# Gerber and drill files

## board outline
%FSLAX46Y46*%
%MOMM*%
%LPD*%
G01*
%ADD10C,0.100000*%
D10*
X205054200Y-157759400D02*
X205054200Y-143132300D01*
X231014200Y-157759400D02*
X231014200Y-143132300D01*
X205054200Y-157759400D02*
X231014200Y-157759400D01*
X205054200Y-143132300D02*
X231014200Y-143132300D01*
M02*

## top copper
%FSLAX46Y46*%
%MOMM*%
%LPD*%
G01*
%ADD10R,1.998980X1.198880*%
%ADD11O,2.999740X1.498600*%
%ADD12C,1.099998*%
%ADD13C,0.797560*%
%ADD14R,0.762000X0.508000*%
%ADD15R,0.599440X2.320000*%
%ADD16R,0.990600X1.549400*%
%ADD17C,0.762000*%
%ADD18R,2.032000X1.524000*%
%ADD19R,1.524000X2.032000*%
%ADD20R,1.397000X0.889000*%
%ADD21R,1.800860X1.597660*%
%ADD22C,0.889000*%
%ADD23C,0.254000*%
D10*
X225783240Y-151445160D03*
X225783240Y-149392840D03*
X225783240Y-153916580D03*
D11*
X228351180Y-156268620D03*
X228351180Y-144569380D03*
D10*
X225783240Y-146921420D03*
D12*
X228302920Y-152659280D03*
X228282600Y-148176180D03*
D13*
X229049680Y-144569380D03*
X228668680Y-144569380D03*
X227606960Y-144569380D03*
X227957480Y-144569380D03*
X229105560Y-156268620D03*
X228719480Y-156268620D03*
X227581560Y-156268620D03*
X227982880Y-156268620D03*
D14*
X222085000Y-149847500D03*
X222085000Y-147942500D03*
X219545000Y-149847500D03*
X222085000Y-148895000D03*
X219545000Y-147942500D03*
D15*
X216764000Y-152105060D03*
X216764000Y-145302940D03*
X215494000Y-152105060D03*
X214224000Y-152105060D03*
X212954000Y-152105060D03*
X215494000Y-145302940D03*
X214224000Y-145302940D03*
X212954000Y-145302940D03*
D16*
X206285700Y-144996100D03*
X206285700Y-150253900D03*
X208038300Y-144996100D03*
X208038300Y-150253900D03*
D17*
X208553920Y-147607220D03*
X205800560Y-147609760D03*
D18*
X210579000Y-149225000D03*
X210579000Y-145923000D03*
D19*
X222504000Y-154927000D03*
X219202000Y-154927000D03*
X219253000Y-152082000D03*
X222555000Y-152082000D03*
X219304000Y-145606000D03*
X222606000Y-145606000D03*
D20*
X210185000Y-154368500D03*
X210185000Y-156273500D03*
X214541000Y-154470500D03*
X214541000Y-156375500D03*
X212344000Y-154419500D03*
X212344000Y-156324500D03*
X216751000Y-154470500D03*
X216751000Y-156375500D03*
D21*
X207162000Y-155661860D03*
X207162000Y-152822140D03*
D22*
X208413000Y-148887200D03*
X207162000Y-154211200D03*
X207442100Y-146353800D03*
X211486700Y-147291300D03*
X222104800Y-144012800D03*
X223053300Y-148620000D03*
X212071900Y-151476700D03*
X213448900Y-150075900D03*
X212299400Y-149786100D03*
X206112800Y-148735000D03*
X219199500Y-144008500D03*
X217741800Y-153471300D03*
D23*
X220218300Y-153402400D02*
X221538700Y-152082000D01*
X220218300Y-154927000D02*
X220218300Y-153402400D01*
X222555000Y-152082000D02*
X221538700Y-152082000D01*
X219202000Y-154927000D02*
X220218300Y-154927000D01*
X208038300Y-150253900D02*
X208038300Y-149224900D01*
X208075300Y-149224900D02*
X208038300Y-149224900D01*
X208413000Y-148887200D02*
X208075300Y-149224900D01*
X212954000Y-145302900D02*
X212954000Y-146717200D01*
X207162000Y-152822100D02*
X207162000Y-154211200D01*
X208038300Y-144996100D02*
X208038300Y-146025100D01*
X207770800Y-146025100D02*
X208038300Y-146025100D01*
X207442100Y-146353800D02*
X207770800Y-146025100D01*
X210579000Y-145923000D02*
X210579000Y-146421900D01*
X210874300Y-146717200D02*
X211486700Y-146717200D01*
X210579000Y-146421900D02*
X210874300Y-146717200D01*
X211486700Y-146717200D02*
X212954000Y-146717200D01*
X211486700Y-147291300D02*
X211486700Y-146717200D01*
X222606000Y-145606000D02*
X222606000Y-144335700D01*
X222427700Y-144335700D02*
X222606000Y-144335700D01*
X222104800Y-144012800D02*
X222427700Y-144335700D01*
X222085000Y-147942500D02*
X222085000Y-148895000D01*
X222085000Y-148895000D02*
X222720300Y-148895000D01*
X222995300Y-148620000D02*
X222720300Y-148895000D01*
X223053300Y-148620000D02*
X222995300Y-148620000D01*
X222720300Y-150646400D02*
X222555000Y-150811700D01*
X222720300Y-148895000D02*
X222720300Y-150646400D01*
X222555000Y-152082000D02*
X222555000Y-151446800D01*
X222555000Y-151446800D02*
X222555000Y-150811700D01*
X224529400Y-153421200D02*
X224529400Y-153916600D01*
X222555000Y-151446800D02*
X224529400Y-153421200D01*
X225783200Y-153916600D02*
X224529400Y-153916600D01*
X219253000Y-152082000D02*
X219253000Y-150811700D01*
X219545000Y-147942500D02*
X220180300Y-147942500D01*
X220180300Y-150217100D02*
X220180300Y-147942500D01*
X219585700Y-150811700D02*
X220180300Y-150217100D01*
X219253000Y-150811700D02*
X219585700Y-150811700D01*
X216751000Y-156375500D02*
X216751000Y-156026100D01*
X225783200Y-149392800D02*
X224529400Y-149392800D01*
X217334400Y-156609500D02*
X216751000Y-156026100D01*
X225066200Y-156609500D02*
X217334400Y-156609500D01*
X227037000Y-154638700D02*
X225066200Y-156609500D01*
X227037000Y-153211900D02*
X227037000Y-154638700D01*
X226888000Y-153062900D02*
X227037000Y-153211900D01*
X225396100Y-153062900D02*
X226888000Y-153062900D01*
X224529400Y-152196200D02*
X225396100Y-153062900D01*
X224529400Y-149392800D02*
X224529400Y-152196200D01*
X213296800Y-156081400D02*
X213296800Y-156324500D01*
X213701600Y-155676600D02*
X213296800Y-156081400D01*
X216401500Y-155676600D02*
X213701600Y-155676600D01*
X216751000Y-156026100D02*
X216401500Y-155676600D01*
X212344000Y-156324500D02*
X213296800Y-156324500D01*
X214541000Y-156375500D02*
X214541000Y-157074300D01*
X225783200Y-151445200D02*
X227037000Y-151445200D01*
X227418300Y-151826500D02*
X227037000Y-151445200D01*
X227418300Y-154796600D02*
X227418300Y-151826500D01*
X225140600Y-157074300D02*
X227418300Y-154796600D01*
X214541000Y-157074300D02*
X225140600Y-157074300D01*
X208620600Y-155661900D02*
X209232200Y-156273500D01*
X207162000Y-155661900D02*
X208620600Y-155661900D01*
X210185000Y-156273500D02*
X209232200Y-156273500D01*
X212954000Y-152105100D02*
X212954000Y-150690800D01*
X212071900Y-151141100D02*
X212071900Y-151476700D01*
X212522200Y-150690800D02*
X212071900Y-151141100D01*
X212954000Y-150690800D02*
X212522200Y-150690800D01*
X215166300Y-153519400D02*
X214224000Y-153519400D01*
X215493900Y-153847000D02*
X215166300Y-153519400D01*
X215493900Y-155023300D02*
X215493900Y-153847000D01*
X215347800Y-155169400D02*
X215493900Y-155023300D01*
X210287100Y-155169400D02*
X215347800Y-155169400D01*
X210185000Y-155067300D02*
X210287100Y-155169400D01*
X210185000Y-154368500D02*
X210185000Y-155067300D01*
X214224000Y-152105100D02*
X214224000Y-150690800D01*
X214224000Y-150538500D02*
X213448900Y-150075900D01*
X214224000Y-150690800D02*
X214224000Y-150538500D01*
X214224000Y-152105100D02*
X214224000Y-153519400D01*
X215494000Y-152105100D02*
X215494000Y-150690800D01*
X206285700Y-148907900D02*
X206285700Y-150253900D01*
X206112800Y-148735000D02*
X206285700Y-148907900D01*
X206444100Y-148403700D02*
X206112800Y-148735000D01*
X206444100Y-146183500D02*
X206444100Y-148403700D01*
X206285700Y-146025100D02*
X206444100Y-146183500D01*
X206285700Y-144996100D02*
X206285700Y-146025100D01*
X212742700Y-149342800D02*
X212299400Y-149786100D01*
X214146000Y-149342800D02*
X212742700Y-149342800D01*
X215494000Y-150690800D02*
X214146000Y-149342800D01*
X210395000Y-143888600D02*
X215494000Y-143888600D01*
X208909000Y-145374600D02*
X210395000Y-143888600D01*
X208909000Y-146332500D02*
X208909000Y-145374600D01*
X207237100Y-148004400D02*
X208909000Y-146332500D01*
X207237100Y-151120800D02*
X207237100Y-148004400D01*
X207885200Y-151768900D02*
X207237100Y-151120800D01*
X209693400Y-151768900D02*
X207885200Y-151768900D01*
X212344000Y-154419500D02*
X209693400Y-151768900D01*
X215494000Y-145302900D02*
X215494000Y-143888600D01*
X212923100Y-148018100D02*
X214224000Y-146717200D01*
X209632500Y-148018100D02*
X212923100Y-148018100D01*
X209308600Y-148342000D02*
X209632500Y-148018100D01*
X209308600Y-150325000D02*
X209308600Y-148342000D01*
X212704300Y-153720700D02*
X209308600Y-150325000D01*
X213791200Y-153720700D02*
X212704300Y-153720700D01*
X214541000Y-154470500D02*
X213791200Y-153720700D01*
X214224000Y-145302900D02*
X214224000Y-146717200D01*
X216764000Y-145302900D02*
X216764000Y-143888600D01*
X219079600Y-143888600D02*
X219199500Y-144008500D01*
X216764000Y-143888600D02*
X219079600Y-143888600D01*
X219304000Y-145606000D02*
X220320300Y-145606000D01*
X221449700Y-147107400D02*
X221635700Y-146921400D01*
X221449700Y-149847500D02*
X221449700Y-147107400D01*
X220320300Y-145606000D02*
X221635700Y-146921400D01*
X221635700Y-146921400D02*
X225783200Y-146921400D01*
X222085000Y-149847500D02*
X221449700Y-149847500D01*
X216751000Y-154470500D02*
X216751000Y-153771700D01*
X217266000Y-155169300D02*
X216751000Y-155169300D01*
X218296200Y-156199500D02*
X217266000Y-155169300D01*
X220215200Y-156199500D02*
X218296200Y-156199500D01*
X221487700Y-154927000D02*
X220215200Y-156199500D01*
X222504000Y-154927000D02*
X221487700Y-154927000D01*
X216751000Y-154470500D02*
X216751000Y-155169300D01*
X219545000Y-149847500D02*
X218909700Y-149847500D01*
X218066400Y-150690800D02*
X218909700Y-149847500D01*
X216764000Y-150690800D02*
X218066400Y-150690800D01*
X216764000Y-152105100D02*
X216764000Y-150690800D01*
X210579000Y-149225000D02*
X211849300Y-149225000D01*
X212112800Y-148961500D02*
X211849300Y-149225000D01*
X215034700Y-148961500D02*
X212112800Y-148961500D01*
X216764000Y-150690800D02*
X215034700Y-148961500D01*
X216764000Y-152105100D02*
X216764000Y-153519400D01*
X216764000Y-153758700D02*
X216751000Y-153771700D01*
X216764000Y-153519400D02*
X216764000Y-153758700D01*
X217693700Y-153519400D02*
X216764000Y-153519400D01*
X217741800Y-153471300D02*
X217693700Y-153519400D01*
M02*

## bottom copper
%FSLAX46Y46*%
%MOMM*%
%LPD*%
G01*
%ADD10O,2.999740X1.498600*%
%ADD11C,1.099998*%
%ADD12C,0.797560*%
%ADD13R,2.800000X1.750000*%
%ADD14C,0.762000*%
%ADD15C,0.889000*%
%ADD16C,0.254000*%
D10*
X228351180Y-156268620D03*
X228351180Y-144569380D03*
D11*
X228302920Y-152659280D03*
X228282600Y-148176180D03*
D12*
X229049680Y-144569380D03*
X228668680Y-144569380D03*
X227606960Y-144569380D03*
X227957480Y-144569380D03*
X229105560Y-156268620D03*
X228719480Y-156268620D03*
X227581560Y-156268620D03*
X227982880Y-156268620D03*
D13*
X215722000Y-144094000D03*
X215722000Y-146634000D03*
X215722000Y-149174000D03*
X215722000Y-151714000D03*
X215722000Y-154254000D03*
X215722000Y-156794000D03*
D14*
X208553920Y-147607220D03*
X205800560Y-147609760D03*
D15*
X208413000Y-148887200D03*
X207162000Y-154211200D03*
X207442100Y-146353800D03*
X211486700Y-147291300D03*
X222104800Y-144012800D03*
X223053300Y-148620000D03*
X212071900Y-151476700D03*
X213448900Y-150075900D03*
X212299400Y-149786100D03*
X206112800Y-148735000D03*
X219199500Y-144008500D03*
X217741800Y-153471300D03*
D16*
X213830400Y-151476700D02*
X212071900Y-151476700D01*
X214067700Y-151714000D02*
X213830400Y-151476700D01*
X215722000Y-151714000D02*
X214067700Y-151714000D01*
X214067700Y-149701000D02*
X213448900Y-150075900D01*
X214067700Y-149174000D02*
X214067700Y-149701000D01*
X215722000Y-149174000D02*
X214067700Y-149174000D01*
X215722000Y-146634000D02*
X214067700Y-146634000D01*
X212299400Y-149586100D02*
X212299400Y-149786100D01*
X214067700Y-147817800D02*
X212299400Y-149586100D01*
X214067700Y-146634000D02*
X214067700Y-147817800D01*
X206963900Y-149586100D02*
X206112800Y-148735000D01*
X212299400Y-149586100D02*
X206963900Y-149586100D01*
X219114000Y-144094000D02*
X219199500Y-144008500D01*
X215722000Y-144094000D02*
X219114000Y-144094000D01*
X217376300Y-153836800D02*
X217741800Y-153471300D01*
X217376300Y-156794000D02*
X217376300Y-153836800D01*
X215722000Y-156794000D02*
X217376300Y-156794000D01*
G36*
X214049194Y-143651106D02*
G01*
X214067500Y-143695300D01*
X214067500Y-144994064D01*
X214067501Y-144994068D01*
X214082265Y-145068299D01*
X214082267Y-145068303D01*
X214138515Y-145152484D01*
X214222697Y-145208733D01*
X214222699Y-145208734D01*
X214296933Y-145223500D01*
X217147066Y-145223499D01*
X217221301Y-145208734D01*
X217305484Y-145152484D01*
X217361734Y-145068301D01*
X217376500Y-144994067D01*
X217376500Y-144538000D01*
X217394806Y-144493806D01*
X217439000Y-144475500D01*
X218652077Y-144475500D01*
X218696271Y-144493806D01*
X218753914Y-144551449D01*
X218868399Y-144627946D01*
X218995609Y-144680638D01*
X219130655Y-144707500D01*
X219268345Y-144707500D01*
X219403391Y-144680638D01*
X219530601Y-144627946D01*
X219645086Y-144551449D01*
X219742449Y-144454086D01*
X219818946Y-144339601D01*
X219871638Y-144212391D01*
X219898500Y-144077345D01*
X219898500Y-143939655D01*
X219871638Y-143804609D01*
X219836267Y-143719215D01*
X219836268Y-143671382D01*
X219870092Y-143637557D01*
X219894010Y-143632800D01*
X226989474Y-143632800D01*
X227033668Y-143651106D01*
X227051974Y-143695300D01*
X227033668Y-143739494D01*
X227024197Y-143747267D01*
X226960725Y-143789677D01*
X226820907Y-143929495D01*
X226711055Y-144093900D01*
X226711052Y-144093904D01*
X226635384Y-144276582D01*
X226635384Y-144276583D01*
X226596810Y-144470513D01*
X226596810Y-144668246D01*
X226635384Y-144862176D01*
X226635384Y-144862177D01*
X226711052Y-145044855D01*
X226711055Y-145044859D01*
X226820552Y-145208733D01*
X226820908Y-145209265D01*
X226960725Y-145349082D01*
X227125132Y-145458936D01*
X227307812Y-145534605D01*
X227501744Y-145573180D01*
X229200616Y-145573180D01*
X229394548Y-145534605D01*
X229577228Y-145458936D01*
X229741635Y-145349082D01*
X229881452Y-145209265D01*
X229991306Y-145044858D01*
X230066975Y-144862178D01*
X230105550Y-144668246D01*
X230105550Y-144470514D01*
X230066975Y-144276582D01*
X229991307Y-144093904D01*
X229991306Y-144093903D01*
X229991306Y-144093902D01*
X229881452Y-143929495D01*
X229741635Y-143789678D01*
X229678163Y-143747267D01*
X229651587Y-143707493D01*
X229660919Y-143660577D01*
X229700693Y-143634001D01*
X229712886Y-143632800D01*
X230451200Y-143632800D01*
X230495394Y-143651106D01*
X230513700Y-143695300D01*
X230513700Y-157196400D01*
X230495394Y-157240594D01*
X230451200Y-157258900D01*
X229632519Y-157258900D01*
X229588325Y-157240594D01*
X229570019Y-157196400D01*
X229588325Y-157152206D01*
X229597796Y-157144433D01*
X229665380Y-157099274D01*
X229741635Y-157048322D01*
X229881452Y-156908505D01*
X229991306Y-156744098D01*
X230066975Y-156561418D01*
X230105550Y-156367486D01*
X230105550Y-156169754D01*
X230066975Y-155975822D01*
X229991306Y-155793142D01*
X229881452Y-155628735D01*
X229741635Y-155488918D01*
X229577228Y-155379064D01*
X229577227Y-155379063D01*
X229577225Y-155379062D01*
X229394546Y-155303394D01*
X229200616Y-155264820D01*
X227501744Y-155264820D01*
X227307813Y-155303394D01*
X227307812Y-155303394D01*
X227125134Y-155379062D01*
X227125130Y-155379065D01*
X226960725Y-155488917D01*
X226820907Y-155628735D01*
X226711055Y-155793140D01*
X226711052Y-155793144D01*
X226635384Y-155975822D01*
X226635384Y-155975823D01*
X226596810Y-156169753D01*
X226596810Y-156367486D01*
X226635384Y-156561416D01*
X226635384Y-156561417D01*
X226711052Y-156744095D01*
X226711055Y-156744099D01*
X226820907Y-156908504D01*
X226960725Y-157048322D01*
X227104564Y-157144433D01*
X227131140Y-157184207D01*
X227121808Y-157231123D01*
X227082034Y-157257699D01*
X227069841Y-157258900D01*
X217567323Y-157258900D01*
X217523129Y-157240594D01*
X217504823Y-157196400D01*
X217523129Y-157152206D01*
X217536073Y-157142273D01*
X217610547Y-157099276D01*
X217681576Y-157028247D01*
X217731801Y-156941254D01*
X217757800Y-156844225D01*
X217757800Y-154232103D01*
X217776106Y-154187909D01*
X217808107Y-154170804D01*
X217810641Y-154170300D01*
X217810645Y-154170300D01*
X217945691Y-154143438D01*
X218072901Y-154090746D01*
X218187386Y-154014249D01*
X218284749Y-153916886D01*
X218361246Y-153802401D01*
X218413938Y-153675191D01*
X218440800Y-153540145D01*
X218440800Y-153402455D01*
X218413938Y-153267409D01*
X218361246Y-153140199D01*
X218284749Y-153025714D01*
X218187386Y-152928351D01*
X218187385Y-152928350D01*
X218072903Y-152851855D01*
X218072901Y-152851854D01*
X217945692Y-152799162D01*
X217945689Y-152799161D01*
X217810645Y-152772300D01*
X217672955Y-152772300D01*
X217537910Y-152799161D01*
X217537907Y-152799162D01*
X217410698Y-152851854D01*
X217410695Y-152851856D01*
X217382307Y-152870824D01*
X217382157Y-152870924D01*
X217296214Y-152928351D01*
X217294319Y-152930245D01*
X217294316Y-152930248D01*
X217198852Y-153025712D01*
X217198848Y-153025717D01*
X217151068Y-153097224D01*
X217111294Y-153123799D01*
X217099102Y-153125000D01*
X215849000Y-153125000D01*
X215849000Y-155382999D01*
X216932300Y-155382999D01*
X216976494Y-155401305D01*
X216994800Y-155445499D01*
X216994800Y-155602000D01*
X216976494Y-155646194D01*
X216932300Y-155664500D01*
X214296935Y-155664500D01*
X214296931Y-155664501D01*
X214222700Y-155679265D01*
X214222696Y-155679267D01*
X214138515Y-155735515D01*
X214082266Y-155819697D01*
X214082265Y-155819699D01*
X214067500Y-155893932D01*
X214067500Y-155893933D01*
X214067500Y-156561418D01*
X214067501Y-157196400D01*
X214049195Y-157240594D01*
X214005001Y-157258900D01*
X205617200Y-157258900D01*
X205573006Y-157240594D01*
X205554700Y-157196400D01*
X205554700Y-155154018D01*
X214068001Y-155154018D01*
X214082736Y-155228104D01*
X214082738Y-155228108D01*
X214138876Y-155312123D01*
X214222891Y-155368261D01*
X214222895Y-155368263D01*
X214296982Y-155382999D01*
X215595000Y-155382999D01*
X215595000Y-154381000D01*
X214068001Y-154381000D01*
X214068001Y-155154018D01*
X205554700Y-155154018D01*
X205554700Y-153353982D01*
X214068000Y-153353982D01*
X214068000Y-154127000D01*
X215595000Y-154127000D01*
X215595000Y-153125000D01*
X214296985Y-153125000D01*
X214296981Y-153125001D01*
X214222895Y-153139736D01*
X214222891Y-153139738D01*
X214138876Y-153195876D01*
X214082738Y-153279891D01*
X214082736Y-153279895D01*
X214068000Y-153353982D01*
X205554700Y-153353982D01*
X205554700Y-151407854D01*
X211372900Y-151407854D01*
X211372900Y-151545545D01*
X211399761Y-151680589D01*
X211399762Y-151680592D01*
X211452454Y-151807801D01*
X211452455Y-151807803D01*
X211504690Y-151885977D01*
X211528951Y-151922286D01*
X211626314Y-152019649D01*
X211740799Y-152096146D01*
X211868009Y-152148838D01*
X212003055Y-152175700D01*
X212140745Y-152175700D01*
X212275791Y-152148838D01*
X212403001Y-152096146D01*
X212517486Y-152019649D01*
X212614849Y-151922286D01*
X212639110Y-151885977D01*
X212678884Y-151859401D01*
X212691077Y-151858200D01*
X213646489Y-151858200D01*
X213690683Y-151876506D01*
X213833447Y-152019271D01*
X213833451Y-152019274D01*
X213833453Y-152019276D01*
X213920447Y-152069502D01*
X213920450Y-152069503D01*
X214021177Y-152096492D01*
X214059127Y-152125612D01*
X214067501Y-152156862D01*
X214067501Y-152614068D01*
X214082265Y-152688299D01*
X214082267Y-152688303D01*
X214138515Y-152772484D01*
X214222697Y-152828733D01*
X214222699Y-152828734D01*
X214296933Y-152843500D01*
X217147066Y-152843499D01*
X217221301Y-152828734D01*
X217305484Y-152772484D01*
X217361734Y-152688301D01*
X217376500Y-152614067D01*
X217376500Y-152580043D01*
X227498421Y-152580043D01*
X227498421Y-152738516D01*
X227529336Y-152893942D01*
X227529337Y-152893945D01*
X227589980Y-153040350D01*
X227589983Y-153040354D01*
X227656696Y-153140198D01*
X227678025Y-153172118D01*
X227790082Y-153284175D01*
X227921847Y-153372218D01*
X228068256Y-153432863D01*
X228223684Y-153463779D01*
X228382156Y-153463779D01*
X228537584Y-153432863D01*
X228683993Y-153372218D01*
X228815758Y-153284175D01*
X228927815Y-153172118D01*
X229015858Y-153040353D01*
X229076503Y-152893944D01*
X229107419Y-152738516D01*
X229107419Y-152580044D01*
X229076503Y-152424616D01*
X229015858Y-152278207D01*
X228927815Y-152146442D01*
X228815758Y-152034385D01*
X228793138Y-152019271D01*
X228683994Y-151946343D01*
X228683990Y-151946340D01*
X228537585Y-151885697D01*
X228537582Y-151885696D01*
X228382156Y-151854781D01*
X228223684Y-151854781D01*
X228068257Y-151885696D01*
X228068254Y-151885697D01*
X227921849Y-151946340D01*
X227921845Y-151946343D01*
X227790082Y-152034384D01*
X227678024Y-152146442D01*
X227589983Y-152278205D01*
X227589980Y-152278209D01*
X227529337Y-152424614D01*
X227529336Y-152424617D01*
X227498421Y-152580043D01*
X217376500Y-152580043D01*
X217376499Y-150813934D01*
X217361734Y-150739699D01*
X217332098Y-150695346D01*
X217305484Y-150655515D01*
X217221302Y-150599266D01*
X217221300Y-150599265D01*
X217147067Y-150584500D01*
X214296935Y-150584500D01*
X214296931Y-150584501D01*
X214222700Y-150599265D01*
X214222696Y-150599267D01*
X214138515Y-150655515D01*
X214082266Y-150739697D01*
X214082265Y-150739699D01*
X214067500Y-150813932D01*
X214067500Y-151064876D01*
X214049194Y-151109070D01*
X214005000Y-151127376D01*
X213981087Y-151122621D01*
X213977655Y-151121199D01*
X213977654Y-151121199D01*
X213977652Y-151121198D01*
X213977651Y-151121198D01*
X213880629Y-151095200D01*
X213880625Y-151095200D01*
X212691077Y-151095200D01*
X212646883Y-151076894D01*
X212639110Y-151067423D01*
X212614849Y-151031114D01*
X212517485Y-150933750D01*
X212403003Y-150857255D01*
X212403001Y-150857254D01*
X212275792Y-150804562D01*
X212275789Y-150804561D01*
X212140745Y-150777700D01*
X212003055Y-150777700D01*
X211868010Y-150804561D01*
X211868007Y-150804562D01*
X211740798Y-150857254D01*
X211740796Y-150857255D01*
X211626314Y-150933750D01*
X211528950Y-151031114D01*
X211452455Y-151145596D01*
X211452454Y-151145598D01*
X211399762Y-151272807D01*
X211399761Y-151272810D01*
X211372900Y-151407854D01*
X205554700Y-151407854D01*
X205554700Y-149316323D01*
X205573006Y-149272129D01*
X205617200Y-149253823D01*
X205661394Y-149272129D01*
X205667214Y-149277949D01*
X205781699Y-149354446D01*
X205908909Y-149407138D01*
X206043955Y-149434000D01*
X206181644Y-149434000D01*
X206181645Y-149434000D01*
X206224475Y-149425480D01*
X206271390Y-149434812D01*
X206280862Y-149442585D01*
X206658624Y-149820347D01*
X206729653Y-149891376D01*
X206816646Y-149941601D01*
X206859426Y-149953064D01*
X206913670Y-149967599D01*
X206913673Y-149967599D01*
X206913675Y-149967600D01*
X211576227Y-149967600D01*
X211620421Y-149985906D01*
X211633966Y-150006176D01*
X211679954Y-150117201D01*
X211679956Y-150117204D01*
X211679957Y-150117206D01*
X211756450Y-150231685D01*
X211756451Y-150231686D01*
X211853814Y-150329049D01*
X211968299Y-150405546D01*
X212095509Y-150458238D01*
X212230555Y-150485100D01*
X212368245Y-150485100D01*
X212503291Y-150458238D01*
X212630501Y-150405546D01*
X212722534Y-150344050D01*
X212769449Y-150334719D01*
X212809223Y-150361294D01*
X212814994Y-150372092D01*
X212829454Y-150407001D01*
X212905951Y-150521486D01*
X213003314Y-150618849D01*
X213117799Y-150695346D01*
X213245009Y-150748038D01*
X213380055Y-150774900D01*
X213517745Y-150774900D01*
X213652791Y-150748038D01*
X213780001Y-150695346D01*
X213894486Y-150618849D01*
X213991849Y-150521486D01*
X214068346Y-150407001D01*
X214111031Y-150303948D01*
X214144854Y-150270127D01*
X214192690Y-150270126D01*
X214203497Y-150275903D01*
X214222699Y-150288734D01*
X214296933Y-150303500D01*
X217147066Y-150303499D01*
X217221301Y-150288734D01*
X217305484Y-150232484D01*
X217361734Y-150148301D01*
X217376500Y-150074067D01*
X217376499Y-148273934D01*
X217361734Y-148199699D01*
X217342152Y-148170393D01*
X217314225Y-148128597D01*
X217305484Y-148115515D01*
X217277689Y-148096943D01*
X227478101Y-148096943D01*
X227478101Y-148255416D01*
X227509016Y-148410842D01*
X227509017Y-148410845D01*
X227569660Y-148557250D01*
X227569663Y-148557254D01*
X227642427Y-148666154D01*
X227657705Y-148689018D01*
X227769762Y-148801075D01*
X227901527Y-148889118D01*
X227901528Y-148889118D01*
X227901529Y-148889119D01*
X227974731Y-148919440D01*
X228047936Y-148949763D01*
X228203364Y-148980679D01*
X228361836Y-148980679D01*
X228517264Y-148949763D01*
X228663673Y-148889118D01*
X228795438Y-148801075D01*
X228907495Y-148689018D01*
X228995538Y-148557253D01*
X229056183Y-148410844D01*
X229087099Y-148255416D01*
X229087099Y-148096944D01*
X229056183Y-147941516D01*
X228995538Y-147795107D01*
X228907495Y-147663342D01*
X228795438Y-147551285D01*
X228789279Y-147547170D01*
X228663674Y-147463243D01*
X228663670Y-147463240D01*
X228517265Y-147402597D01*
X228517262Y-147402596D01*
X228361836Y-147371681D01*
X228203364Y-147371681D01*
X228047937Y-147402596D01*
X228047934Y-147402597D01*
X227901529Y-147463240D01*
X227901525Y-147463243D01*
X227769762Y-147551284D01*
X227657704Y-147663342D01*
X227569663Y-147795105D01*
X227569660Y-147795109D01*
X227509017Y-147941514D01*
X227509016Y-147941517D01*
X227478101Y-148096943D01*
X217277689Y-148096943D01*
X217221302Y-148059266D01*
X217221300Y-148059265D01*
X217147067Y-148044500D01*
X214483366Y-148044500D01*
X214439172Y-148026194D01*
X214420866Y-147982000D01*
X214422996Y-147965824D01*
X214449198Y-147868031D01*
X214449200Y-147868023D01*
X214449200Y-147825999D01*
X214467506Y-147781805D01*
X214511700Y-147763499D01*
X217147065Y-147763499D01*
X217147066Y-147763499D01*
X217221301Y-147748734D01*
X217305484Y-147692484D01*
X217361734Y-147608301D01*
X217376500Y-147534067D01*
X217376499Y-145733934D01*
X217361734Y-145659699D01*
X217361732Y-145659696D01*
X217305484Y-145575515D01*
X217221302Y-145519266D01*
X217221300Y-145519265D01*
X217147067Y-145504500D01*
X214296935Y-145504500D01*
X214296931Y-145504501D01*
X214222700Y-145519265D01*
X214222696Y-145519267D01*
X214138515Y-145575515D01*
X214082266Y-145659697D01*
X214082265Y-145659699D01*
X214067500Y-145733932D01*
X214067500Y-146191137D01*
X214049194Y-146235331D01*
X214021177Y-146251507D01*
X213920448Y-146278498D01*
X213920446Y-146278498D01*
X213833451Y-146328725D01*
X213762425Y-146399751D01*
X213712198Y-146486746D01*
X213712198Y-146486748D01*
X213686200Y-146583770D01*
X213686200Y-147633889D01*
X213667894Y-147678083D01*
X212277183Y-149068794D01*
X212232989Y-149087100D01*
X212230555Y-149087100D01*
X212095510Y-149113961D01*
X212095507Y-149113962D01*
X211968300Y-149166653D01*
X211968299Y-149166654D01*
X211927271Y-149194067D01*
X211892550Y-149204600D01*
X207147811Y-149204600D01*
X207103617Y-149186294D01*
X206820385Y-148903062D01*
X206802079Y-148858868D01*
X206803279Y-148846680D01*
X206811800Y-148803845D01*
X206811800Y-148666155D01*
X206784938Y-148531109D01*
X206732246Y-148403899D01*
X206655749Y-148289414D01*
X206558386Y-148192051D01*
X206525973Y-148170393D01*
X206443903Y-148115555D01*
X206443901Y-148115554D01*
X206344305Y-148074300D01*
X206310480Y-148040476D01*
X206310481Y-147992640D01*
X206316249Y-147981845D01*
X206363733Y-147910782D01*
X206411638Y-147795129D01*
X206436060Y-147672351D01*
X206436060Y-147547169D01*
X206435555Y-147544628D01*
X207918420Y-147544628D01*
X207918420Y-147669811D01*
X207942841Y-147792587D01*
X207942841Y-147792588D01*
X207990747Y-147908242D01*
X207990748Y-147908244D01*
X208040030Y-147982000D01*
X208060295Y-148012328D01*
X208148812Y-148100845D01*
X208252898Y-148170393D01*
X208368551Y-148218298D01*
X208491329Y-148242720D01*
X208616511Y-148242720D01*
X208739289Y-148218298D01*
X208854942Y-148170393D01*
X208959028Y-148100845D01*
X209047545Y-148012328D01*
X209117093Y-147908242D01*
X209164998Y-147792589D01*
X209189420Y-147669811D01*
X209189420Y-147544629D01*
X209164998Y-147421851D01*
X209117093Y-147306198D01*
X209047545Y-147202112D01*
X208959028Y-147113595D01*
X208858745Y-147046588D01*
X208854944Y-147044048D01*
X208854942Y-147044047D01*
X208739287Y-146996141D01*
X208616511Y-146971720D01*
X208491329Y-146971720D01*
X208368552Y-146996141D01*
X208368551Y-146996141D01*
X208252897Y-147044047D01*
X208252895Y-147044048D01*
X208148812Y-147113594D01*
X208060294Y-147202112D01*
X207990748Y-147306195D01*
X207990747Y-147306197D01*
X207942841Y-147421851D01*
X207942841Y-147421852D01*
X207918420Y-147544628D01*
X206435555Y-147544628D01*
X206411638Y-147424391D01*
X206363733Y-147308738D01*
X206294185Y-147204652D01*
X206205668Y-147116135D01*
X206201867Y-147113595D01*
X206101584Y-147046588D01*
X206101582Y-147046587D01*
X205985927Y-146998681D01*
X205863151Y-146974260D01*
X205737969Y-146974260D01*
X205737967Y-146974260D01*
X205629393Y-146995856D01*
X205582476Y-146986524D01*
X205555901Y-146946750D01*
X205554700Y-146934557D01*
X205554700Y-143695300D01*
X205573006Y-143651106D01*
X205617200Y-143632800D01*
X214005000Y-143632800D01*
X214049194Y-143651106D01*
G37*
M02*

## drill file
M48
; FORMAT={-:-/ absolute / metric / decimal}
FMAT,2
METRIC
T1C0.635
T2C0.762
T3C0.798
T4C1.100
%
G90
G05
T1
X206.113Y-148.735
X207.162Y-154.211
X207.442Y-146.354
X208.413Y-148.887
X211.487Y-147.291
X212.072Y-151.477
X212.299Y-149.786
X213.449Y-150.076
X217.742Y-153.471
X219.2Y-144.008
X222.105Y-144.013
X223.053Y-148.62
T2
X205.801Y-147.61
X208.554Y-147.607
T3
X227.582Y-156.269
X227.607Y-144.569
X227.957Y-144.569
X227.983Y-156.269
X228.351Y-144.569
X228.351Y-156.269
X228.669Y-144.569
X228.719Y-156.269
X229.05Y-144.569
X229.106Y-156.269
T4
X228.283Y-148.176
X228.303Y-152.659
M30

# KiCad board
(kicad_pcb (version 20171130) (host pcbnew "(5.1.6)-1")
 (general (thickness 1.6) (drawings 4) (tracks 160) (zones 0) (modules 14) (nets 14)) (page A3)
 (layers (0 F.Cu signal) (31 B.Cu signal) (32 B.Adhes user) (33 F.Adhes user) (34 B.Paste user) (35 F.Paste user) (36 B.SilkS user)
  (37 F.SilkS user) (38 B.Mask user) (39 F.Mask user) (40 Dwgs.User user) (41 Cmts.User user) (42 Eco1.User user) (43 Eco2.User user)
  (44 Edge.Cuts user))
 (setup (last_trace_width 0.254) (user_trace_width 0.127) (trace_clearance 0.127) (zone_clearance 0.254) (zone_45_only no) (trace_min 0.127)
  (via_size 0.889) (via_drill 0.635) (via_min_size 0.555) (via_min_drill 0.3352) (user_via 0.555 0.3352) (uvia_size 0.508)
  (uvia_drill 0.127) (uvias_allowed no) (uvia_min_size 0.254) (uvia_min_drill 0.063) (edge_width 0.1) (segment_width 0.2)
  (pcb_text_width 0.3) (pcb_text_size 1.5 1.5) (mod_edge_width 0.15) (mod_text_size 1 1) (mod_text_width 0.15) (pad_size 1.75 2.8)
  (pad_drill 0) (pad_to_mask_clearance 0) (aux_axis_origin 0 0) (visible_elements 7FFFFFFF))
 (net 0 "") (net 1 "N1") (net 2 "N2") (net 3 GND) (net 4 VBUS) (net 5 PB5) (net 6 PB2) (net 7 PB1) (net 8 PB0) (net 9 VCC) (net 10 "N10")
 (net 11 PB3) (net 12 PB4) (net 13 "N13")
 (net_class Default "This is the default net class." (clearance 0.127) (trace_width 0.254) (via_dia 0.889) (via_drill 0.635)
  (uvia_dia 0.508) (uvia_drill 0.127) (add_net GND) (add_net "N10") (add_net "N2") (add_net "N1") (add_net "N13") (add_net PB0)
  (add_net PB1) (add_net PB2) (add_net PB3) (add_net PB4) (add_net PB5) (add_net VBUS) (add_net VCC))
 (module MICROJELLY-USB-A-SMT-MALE (layer F.Cu) (at 229.451 150.419 270)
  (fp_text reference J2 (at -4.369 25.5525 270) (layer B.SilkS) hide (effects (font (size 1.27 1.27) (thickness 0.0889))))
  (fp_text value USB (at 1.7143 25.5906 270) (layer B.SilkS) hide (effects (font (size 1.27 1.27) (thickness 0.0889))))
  (pad 2 smd rect (at 1.02616 3.66776 270) (size 1.19888 1.99898) (layers F.Cu F.Paste F.Mask) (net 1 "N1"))
  (pad 3 smd rect (at -1.02616 3.66776 270) (size 1.19888 1.99898) (layers F.Cu F.Paste F.Mask) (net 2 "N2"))
  (pad 1 smd rect (at 3.49758 3.66776 270) (size 1.19888 1.99898) (layers F.Cu F.Paste F.Mask) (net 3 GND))
  (pad P$1 thru_hole oval (at 5.84962 1.09982 270) (size 1.4986 2.99974) (drill 0.79756) (layers *.Cu *.Mask F.Paste F.SilkS))
  (pad P$3 thru_hole oval (at -5.84962 1.09982 270) (size 1.4986 2.99974) (drill 0.79756) (layers *.Cu *.Mask F.Paste F.SilkS))
  (pad 4 smd rect (at -3.49758 3.66776 270) (size 1.19888 1.99898) (layers F.Cu F.Paste F.Mask) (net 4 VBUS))
  (pad P$4 thru_hole circle (at 2.24028 1.14808 270) (size 1.099998 1.099998) (drill 1.099998) (layers *.Cu *.Mask F.SilkS))
  (pad P$5 thru_hole circle (at -2.24282 1.1684 270) (size 1.099998 1.099998) (drill 1.099998) (layers *.Cu *.Mask F.SilkS))
  (pad P$4 thru_hole circle (at -5.84962 0.40132 270) (size 0.79756 0.79756) (drill 0.79756) (layers *.Cu F.Paste F.SilkS F.Mask))
  (pad P$5 thru_hole circle (at -5.84962 0.78232 270) (size 0.79756 0.79756) (drill 0.79756) (layers *.Cu F.Paste F.SilkS F.Mask))
  (pad P$6 thru_hole circle (at -5.84962 1.84404 270) (size 0.79756 0.79756) (drill 0.79756) (layers *.Cu F.Paste F.SilkS F.Mask))
  (pad P$7 thru_hole circle (at -5.84962 1.49352 270) (size 0.79756 0.79756) (drill 0.79756) (layers *.Cu F.Paste F.SilkS F.Mask))
  (pad P$2 thru_hole circle (at 5.84962 0.34544 270) (size 0.79756 0.79756) (drill 0.79756) (layers *.Cu F.Paste F.SilkS F.Mask))
  (pad P$3 thru_hole circle (at 5.84962 0.73152 270) (size 0.79756 0.79756) (drill 0.79756) (layers *.Cu F.Paste F.SilkS F.Mask))
  (pad P$4 thru_hole circle (at 5.84962 1.86944 270) (size 0.79756 0.79756) (drill 0.79756) (layers *.Cu F.Paste F.SilkS F.Mask))
  (pad P$5 thru_hole circle (at 5.84962 1.46812 270) (size 0.79756 0.79756) (drill 0.79756) (layers *.Cu F.Paste F.SilkS F.Mask)))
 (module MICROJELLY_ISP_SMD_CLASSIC (layer B.Cu) (at 213.944 150.444 270)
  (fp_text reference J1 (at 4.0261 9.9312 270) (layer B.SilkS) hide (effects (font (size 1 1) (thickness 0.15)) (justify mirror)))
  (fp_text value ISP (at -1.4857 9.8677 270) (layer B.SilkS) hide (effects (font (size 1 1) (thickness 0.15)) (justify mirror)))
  (pad 5 smd rect (at -6.35 -1.778 270) (size 1.75 2.8) (layers B.Cu B.Paste B.Mask) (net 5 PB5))
  (pad 3 smd rect (at -3.81 -1.778 270) (size 1.75 2.8) (layers B.Cu B.Paste B.Mask) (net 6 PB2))
  (pad 1 smd rect (at -1.27 -1.778 270) (size 1.75 2.8) (layers B.Cu B.Paste B.Mask) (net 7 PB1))
  (pad 4 smd rect (at 1.27 -1.778 270) (size 1.75 2.8) (layers B.Cu B.Paste B.Mask) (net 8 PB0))
  (pad 6 smd rect (at 3.81 -1.778 270) (size 1.75 2.8) (layers B.Cu B.Paste B.Mask) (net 3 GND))
  (pad 2 smd rect (at 6.35 -1.778 270) (size 1.75 2.8) (layers B.Cu B.Paste B.Mask) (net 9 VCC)))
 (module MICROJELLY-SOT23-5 (layer F.Cu) (at 220.815 148.895 90)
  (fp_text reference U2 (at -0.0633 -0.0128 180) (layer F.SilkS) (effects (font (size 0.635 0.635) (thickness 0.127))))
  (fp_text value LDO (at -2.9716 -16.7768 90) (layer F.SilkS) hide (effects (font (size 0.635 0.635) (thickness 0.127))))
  (pad 1 smd rect (at -0.9525 1.27 90) (size 0.508 0.762) (layers F.Cu F.Paste F.Mask) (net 4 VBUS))
  (pad 3 smd rect (at 0.9525 1.27 90) (size 0.508 0.762) (layers F.Cu F.Paste F.Mask) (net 3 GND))
  (pad 5 smd rect (at -0.9525 -1.27 90) (size 0.508 0.762) (layers F.Cu F.Paste F.Mask) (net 9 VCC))
  (pad 2 smd rect (at 0 1.27 90) (size 0.508 0.762) (layers F.Cu F.Paste F.Mask) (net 3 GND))
  (pad 4 smd rect (at 0.9525 -1.27 90) (size 0.508 0.762) (layers F.Cu F.Paste F.Mask) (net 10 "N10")))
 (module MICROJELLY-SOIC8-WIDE (layer F.Cu) (at 214.859 148.704 180)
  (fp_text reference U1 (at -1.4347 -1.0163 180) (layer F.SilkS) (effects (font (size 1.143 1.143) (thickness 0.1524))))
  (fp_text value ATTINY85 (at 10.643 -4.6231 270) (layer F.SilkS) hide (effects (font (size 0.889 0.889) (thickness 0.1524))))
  (pad 8 smd rect (at -1.905 -3.40106 180) (size 0.59944 2.32) (layers F.Cu F.Paste F.Mask) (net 9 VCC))
  (pad 1 smd rect (at -1.905 3.40106 180) (size 0.59944 2.32) (layers F.Cu F.Paste F.Mask) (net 5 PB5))
  (pad 7 smd rect (at -0.635 -3.40106 180) (size 0.59944 2.32) (layers F.Cu F.Paste F.Mask) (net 6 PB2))
  (pad 6 smd rect (at 0.635 -3.40106 180) (size 0.59944 2.32) (layers F.Cu F.Paste F.Mask) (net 7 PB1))
  (pad 5 smd rect (at 1.905 -3.40106 180) (size 0.59944 2.32) (layers F.Cu F.Paste F.Mask) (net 8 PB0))
  (pad 2 smd rect (at -0.635 3.40106 180) (size 0.59944 2.32) (layers F.Cu F.Paste F.Mask) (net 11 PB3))
  (pad 3 smd rect (at 0.635 3.40106 180) (size 0.59944 2.32) (layers F.Cu F.Paste F.Mask) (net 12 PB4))
  (pad 4 smd rect (at 1.905 3.40106 180) (size 0.59944 2.32) (layers F.Cu F.Paste F.Mask) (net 3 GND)))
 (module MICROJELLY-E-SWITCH (layer F.Cu) (at 207.162 147.625 270)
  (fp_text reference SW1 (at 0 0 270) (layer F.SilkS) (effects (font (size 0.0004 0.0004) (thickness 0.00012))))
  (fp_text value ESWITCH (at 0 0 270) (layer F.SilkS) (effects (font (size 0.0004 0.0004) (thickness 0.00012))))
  (pad 1 smd rect (at -2.6289 0.8763 270) (size 1.5494 0.9906) (layers F.Cu F.Paste F.Mask) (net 6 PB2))
  (pad 1 smd rect (at 2.6289 0.8763 270) (size 1.5494 0.9906) (layers F.Cu F.Paste F.Mask) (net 6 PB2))
  (pad 2 smd rect (at -2.6289 -0.8763 270) (size 1.5494 0.9906) (layers F.Cu F.Paste F.Mask) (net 3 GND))
  (pad 2 smd rect (at 2.6289 -0.8763 270) (size 1.5494 0.9906) (layers F.Cu F.Paste F.Mask) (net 3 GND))
  (pad P$5 thru_hole circle (at -0.01778 -1.39192 270) (size 0.762 0.762) (drill 0.762) (layers *.Cu *.Mask F.SilkS))
  (pad P$6 thru_hole circle (at -0.01524 1.36144 270) (size 0.762 0.762) (drill 0.762) (layers *.Cu *.Mask F.SilkS)))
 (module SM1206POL (layer F.Cu) (at 210.579 147.574 90)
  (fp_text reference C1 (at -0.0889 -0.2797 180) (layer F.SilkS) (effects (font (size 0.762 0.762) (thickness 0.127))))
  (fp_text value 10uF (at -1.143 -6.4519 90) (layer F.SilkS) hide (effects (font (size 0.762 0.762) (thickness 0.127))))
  (pad 1 smd rect (at -1.651 0 90) (size 1.524 2.032) (layers F.Cu F.Paste F.Mask) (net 9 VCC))
  (pad 2 smd rect (at 1.651 0 90) (size 1.524 2.032) (layers F.Cu F.Paste F.Mask) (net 3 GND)))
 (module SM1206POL (layer F.Cu) (at 220.853 154.927 180)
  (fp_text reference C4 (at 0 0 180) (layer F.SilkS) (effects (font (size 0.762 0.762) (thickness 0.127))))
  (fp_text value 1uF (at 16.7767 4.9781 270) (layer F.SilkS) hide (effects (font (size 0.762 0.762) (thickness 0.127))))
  (pad 1 smd rect (at -1.651 0 180) (size 1.524 2.032) (layers F.Cu F.Paste F.Mask) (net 9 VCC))
  (pad 2 smd rect (at 1.651 0 180) (size 1.524 2.032) (layers F.Cu F.Paste F.Mask) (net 3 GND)))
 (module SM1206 (layer F.Cu) (at 220.904 152.082)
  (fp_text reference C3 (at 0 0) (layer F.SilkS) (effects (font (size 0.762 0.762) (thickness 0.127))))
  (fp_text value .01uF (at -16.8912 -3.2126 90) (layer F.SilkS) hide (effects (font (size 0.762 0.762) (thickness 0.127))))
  (pad 1 smd rect (at -1.651 0) (size 1.524 2.032) (layers F.Cu F.Paste F.Mask) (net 10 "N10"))
  (pad 2 smd rect (at 1.651 0) (size 1.524 2.032) (layers F.Cu F.Paste F.Mask) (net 3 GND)))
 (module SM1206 (layer F.Cu) (at 220.955 145.606)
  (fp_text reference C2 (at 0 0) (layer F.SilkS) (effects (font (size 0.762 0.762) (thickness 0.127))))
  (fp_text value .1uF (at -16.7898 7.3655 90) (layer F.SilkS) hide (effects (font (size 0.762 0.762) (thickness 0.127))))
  (pad 1 smd rect (at -1.651 0) (size 1.524 2.032) (layers F.Cu F.Paste F.Mask) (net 4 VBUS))
  (pad 2 smd rect (at 1.651 0) (size 1.524 2.032) (layers F.Cu F.Paste F.Mask) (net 3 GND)))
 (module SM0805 (layer F.Cu) (at 210.185 155.321 270)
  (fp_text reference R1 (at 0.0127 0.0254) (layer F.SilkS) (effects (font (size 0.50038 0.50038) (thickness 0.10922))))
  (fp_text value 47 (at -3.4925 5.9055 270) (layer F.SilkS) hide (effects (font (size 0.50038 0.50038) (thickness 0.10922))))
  (pad 1 smd rect (at -0.9525 0 270) (size 0.889 1.397) (layers F.Cu F.Paste F.Mask) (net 7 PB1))
  (pad 2 smd rect (at 0.9525 0 270) (size 0.889 1.397) (layers F.Cu F.Paste F.Mask) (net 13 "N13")))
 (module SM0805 (layer F.Cu) (at 214.541 155.423 270)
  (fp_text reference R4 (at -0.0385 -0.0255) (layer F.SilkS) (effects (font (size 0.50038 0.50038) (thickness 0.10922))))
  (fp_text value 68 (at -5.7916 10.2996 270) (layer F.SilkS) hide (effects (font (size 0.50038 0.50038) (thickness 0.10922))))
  (pad 1 smd rect (at -0.9525 0 270) (size 0.889 1.397) (layers F.Cu F.Paste F.Mask) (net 12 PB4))
  (pad 2 smd rect (at 0.9525 0 270) (size 0.889 1.397) (layers F.Cu F.Paste F.Mask) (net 1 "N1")))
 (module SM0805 (layer F.Cu) (at 212.344 155.372 270)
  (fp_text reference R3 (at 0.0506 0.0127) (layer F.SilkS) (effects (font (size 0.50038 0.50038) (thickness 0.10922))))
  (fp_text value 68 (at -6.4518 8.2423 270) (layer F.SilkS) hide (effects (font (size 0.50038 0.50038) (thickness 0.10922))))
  (pad 1 smd rect (at -0.9525 0 270) (size 0.889 1.397) (layers F.Cu F.Paste F.Mask) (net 11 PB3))
  (pad 2 smd rect (at 0.9525 0 270) (size 0.889 1.397) (layers F.Cu F.Paste F.Mask) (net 2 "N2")))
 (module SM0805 (layer F.Cu) (at 216.751 155.423 270)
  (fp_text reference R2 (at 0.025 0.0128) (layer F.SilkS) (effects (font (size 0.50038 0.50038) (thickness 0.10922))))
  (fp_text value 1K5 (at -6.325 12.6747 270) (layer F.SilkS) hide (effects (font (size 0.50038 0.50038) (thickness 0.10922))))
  (pad 1 smd rect (at -0.9525 0 270) (size 0.889 1.397) (layers F.Cu F.Paste F.Mask) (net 9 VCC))
  (pad 2 smd rect (at 0.9525 0 270) (size 0.889 1.397) (layers F.Cu F.Paste F.Mask) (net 2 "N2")))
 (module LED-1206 (layer F.Cu) (at 207.162 154.242 90)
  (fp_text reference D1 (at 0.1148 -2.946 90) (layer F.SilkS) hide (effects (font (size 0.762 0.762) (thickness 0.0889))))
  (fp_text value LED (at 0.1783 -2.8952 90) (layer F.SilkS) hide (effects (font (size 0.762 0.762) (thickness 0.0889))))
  (pad 1 smd rect (at -1.41986 0 90) (size 1.59766 1.80086) (layers F.Cu F.Paste F.Mask) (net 13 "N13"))
  (pad 2 smd rect (at 1.41986 0 90) (size 1.59766 1.80086) (layers F.Cu F.Paste F.Mask) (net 3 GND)))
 (gr_line (start 205.0542 157.7594) (end 205.0542 143.1323) (angle 90) (layer Edge.Cuts) (width 0.1))
 (gr_line (start 231.0142 157.7594) (end 231.0142 143.1323) (angle 90) (layer Edge.Cuts) (width 0.1))
 (gr_line (start 205.0542 157.7594) (end 231.0142 157.7594) (angle 90) (layer Edge.Cuts) (width 0.1))
 (gr_line (start 205.0542 143.1323) (end 231.0142 143.1323) (angle 90) (layer Edge.Cuts) (width 0.1))
 (via (at 208.413 148.8872) (size 0.889) (layers F.Cu B.Cu) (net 3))
 (via (at 207.162 154.2112) (size 0.889) (layers F.Cu B.Cu) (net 3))
 (via (at 207.4421 146.3538) (size 0.889) (layers F.Cu B.Cu) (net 3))
 (via (at 211.4867 147.2913) (size 0.889) (layers F.Cu B.Cu) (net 3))
 (via (at 222.1048 144.0128) (size 0.889) (layers F.Cu B.Cu) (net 3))
 (via (at 223.0533 148.62) (size 0.889) (layers F.Cu B.Cu) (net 3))
 (segment (start 220.2183 153.4024) (end 221.5387 152.082) (width 0.254) (layer F.Cu) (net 3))
 (segment (start 220.2183 154.927) (end 220.2183 153.4024) (width 0.254) (layer F.Cu) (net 3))
 (segment (start 222.555 152.082) (end 221.5387 152.082) (width 0.254) (layer F.Cu) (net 3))
 (segment (start 219.202 154.927) (end 220.2183 154.927) (width 0.254) (layer F.Cu) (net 3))
 (segment (start 208.0383 150.2539) (end 208.0383 149.2249) (width 0.254) (layer F.Cu) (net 3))
 (segment (start 208.0753 149.2249) (end 208.0383 149.2249) (width 0.254) (layer F.Cu) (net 3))
 (segment (start 208.413 148.8872) (end 208.0753 149.2249) (width 0.254) (layer F.Cu) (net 3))
 (segment (start 212.954 145.3029) (end 212.954 146.7172) (width 0.254) (layer F.Cu) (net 3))
 (segment (start 207.162 152.8221) (end 207.162 154.2112) (width 0.254) (layer F.Cu) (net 3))
 (segment (start 208.0383 144.9961) (end 208.0383 146.0251) (width 0.254) (layer F.Cu) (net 3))
 (segment (start 207.7708 146.0251) (end 208.0383 146.0251) (width 0.254) (layer F.Cu) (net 3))
 (segment (start 207.4421 146.3538) (end 207.7708 146.0251) (width 0.254) (layer F.Cu) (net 3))
 (segment (start 210.579 145.923) (end 210.579 146.4219) (width 0.254) (layer F.Cu) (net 3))
 (segment (start 210.8743 146.7172) (end 211.4867 146.7172) (width 0.254) (layer F.Cu) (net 3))
 (segment (start 210.579 146.4219) (end 210.8743 146.7172) (width 0.254) (layer F.Cu) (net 3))
 (segment (start 211.4867 146.7172) (end 212.954 146.7172) (width 0.254) (layer F.Cu) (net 3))
 (segment (start 211.4867 147.2913) (end 211.4867 146.7172) (width 0.254) (layer F.Cu) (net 3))
 (segment (start 222.606 145.606) (end 222.606 144.3357) (width 0.254) (layer F.Cu) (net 3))
 (segment (start 222.4277 144.3357) (end 222.606 144.3357) (width 0.254) (layer F.Cu) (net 3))
 (segment (start 222.1048 144.0128) (end 222.4277 144.3357) (width 0.254) (layer F.Cu) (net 3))
 (segment (start 222.085 147.9425) (end 222.085 148.895) (width 0.254) (layer F.Cu) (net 3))
 (segment (start 222.085 148.895) (end 222.7203 148.895) (width 0.254) (layer F.Cu) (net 3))
 (segment (start 222.9953 148.62) (end 222.7203 148.895) (width 0.254) (layer F.Cu) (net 3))
 (segment (start 223.0533 148.62) (end 222.9953 148.62) (width 0.254) (layer F.Cu) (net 3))
 (segment (start 222.7203 150.6464) (end 222.555 150.8117) (width 0.254) (layer F.Cu) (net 3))
 (segment (start 222.7203 148.895) (end 222.7203 150.6464) (width 0.254) (layer F.Cu) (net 3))
 (segment (start 222.555 152.082) (end 222.555 151.4468) (width 0.254) (layer F.Cu) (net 3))
 (segment (start 222.555 151.4468) (end 222.555 150.8117) (width 0.254) (layer F.Cu) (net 3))
 (segment (start 224.5294 153.4212) (end 224.5294 153.9166) (width 0.254) (layer F.Cu) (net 3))
 (segment (start 222.555 151.4468) (end 224.5294 153.4212) (width 0.254) (layer F.Cu) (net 3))
 (segment (start 225.7832 153.9166) (end 224.5294 153.9166) (width 0.254) (layer F.Cu) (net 3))
 (segment (start 219.253 152.082) (end 219.253 150.8117) (width 0.254) (layer F.Cu) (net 10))
 (segment (start 219.545 147.9425) (end 220.1803 147.9425) (width 0.254) (layer F.Cu) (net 10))
 (segment (start 220.1803 150.2171) (end 220.1803 147.9425) (width 0.254) (layer F.Cu) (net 10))
 (segment (start 219.5857 150.8117) (end 220.1803 150.2171) (width 0.254) (layer F.Cu) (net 10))
 (segment (start 219.253 150.8117) (end 219.5857 150.8117) (width 0.254) (layer F.Cu) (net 10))
 (segment (start 216.751 156.3755) (end 216.751 156.0261) (width 0.254) (layer F.Cu) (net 2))
 (segment (start 225.7832 149.3928) (end 224.5294 149.3928) (width 0.254) (layer F.Cu) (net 2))
 (segment (start 217.3344 156.6095) (end 216.751 156.0261) (width 0.254) (layer F.Cu) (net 2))
 (segment (start 225.0662 156.6095) (end 217.3344 156.6095) (width 0.254) (layer F.Cu) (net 2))
 (segment (start 227.037 154.6387) (end 225.0662 156.6095) (width 0.254) (layer F.Cu) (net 2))
 (segment (start 227.037 153.2119) (end 227.037 154.6387) (width 0.254) (layer F.Cu) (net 2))
 (segment (start 226.888 153.0629) (end 227.037 153.2119) (width 0.254) (layer F.Cu) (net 2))
 (segment (start 225.3961 153.0629) (end 226.888 153.0629) (width 0.254) (layer F.Cu) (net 2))
 (segment (start 224.5294 152.1962) (end 225.3961 153.0629) (width 0.254) (layer F.Cu) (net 2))
 (segment (start 224.5294 149.3928) (end 224.5294 152.1962) (width 0.254) (layer F.Cu) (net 2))
 (segment (start 213.2968 156.0814) (end 213.2968 156.3245) (width 0.254) (layer F.Cu) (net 2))
 (segment (start 213.7016 155.6766) (end 213.2968 156.0814) (width 0.254) (layer F.Cu) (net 2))
 (segment (start 216.4015 155.6766) (end 213.7016 155.6766) (width 0.254) (layer F.Cu) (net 2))
 (segment (start 216.751 156.0261) (end 216.4015 155.6766) (width 0.254) (layer F.Cu) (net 2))
 (segment (start 212.344 156.3245) (end 213.2968 156.3245) (width 0.254) (layer F.Cu) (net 2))
 (segment (start 214.541 156.3755) (end 214.541 157.0743) (width 0.254) (layer F.Cu) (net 1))
 (segment (start 225.7832 151.4452) (end 227.037 151.4452) (width 0.254) (layer F.Cu) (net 1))
 (segment (start 227.4183 151.8265) (end 227.037 151.4452) (width 0.254) (layer F.Cu) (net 1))
 (segment (start 227.4183 154.7966) (end 227.4183 151.8265) (width 0.254) (layer F.Cu) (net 1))
 (segment (start 225.1406 157.0743) (end 227.4183 154.7966) (width 0.254) (layer F.Cu) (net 1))
 (segment (start 214.541 157.0743) (end 225.1406 157.0743) (width 0.254) (layer F.Cu) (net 1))
 (segment (start 208.6206 155.6619) (end 209.2322 156.2735) (width 0.254) (layer F.Cu) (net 13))
 (segment (start 207.162 155.6619) (end 208.6206 155.6619) (width 0.254) (layer F.Cu) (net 13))
 (segment (start 210.185 156.2735) (end 209.2322 156.2735) (width 0.254) (layer F.Cu) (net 13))
 (via (at 212.0719 151.4767) (size 0.889) (layers F.Cu B.Cu) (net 8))
 (segment (start 212.954 152.1051) (end 212.954 150.6908) (width 0.254) (layer F.Cu) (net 8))
 (segment (start 213.8304 151.4767) (end 212.0719 151.4767) (width 0.254) (layer B.Cu) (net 8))
 (segment (start 214.0677 151.714) (end 213.8304 151.4767) (width 0.254) (layer B.Cu) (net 8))
 (segment (start 212.0719 151.1411) (end 212.0719 151.4767) (width 0.254) (layer F.Cu) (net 8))
 (segment (start 212.5222 150.6908) (end 212.0719 151.1411) (width 0.254) (layer F.Cu) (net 8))
 (segment (start 212.954 150.6908) (end 212.5222 150.6908) (width 0.254) (layer F.Cu) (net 8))
 (segment (start 215.722 151.714) (end 214.0677 151.714) (width 0.254) (layer B.Cu) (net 8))
 (via (at 213.4489 150.0759) (size 0.889) (layers F.Cu B.Cu) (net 7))
 (segment (start 215.1663 153.5194) (end 214.224 153.5194) (width 0.254) (layer F.Cu) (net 7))
 (segment (start 215.4939 153.847) (end 215.1663 153.5194) (width 0.254) (layer F.Cu) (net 7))
 (segment (start 215.4939 155.0233) (end 215.4939 153.847) (width 0.254) (layer F.Cu) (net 7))
 (segment (start 215.3478 155.1694) (end 215.4939 155.0233) (width 0.254) (layer F.Cu) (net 7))
 (segment (start 210.2871 155.1694) (end 215.3478 155.1694) (width 0.254) (layer F.Cu) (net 7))
 (segment (start 210.185 155.0673) (end 210.2871 155.1694) (width 0.254) (layer F.Cu) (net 7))
 (segment (start 210.185 154.3685) (end 210.185 155.0673) (width 0.254) (layer F.Cu) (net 7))
 (segment (start 214.224 152.1051) (end 214.224 150.6908) (width 0.254) (layer F.Cu) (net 7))
 (segment (start 214.0677 149.701) (end 213.4489 150.0759) (width 0.254) (layer B.Cu) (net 7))
 (segment (start 214.0677 149.174) (end 214.0677 149.701) (width 0.254) (layer B.Cu) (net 7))
 (segment (start 214.224 150.5385) (end 213.4489 150.0759) (width 0.254) (layer F.Cu) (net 7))
 (segment (start 214.224 150.6908) (end 214.224 150.5385) (width 0.254) (layer F.Cu) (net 7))
 (segment (start 215.722 149.174) (end 214.0677 149.174) (width 0.254) (layer B.Cu) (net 7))
 (segment (start 214.224 152.1051) (end 214.224 153.5194) (width 0.254) (layer F.Cu) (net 7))
 (via (at 212.2994 149.7861) (size 0.889) (layers F.Cu B.Cu) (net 6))
 (via (at 206.1128 148.735) (size 0.889) (layers F.Cu B.Cu) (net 6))
 (segment (start 215.494 152.1051) (end 215.494 150.6908) (width 0.254) (layer F.Cu) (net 6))
 (segment (start 215.722 146.634) (end 214.0677 146.634) (width 0.254) (layer B.Cu) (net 6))
 (segment (start 212.2994 149.5861) (end 212.2994 149.7861) (width 0.254) (layer B.Cu) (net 6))
 (segment (start 214.0677 147.8178) (end 212.2994 149.5861) (width 0.254) (layer B.Cu) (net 6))
 (segment (start 214.0677 146.634) (end 214.0677 147.8178) (width 0.254) (layer B.Cu) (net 6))
 (segment (start 206.9639 149.5861) (end 206.1128 148.735) (width 0.254) (layer B.Cu) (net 6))
 (segment (start 212.2994 149.5861) (end 206.9639 149.5861) (width 0.254) (layer B.Cu) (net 6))
 (segment (start 206.2857 148.9079) (end 206.2857 150.2539) (width 0.254) (layer F.Cu) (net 6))
 (segment (start 206.1128 148.735) (end 206.2857 148.9079) (width 0.254) (layer F.Cu) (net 6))
 (segment (start 206.4441 148.4037) (end 206.1128 148.735) (width 0.254) (layer F.Cu) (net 6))
 (segment (start 206.4441 146.1835) (end 206.4441 148.4037) (width 0.254) (layer F.Cu) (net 6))
 (segment (start 206.2857 146.0251) (end 206.4441 146.1835) (width 0.254) (layer F.Cu) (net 6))
 (segment (start 206.2857 144.9961) (end 206.2857 146.0251) (width 0.254) (layer F.Cu) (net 6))
 (segment (start 212.7427 149.3428) (end 212.2994 149.7861) (width 0.254) (layer F.Cu) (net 6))
 (segment (start 214.146 149.3428) (end 212.7427 149.3428) (width 0.254) (layer F.Cu) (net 6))
 (segment (start 215.494 150.6908) (end 214.146 149.3428) (width 0.254) (layer F.Cu) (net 6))
 (segment (start 210.395 143.8886) (end 215.494 143.8886) (width 0.254) (layer F.Cu) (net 11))
 (segment (start 208.909 145.3746) (end 210.395 143.8886) (width 0.254) (layer F.Cu) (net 11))
 (segment (start 208.909 146.3325) (end 208.909 145.3746) (width 0.254) (layer F.Cu) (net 11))
 (segment (start 207.2371 148.0044) (end 208.909 146.3325) (width 0.254) (layer F.Cu) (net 11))
 (segment (start 207.2371 151.1208) (end 207.2371 148.0044) (width 0.254) (layer F.Cu) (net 11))
 (segment (start 207.8852 151.7689) (end 207.2371 151.1208) (width 0.254) (layer F.Cu) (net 11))
 (segment (start 209.6934 151.7689) (end 207.8852 151.7689) (width 0.254) (layer F.Cu) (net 11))
 (segment (start 212.344 154.4195) (end 209.6934 151.7689) (width 0.254) (layer F.Cu) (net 11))
 (segment (start 215.494 145.3029) (end 215.494 143.8886) (width 0.254) (layer F.Cu) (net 11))
 (segment (start 212.9231 148.0181) (end 214.224 146.7172) (width 0.254) (layer F.Cu) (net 12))
 (segment (start 209.6325 148.0181) (end 212.9231 148.0181) (width 0.254) (layer F.Cu) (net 12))
 (segment (start 209.3086 148.342) (end 209.6325 148.0181) (width 0.254) (layer F.Cu) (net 12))
 (segment (start 209.3086 150.325) (end 209.3086 148.342) (width 0.254) (layer F.Cu) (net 12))
 (segment (start 212.7043 153.7207) (end 209.3086 150.325) (width 0.254) (layer F.Cu) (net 12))
 (segment (start 213.7912 153.7207) (end 212.7043 153.7207) (width 0.254) (layer F.Cu) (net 12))
 (segment (start 214.541 154.4705) (end 213.7912 153.7207) (width 0.254) (layer F.Cu) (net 12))
 (segment (start 214.224 145.3029) (end 214.224 146.7172) (width 0.254) (layer F.Cu) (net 12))
 (via (at 219.1995 144.0085) (size 0.889) (layers F.Cu B.Cu) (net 5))
 (segment (start 216.764 145.3029) (end 216.764 143.8886) (width 0.254) (layer F.Cu) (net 5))
 (segment (start 219.114 144.094) (end 219.1995 144.0085) (width 0.254) (layer B.Cu) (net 5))
 (segment (start 215.722 144.094) (end 219.114 144.094) (width 0.254) (layer B.Cu) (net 5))
 (segment (start 219.0796 143.8886) (end 219.1995 144.0085) (width 0.254) (layer F.Cu) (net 5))
 (segment (start 216.764 143.8886) (end 219.0796 143.8886) (width 0.254) (layer F.Cu) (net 5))
 (segment (start 219.304 145.606) (end 220.3203 145.606) (width 0.254) (layer F.Cu) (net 4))
 (segment (start 221.4497 147.1074) (end 221.6357 146.9214) (width 0.254) (layer F.Cu) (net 4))
 (segment (start 221.4497 149.8475) (end 221.4497 147.1074) (width 0.254) (layer F.Cu) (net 4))
 (segment (start 220.3203 145.606) (end 221.6357 146.9214) (width 0.254) (layer F.Cu) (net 4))
 (segment (start 221.6357 146.9214) (end 225.7832 146.9214) (width 0.254) (layer F.Cu) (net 4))
 (segment (start 222.085 149.8475) (end 221.4497 149.8475) (width 0.254) (layer F.Cu) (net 4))
 (via (at 217.7418 153.4713) (size 0.889) (layers F.Cu B.Cu) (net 9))
 (segment (start 216.751 154.4705) (end 216.751 153.7717) (width 0.254) (layer F.Cu) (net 9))
 (segment (start 217.266 155.1693) (end 216.751 155.1693) (width 0.254) (layer F.Cu) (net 9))
 (segment (start 218.2962 156.1995) (end 217.266 155.1693) (width 0.254) (layer F.Cu) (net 9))
 (segment (start 220.2152 156.1995) (end 218.2962 156.1995) (width 0.254) (layer F.Cu) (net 9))
 (segment (start 221.4877 154.927) (end 220.2152 156.1995) (width 0.254) (layer F.Cu) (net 9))
 (segment (start 222.504 154.927) (end 221.4877 154.927) (width 0.254) (layer F.Cu) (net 9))
 (segment (start 216.751 154.4705) (end 216.751 155.1693) (width 0.254) (layer F.Cu) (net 9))
 (segment (start 219.545 149.8475) (end 218.9097 149.8475) (width 0.254) (layer F.Cu) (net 9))
 (segment (start 218.0664 150.6908) (end 218.9097 149.8475) (width 0.254) (layer F.Cu) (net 9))
 (segment (start 216.764 150.6908) (end 218.0664 150.6908) (width 0.254) (layer F.Cu) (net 9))
 (segment (start 216.764 152.1051) (end 216.764 150.6908) (width 0.254) (layer F.Cu) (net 9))
 (segment (start 210.579 149.225) (end 211.8493 149.225) (width 0.254) (layer F.Cu) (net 9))
 (segment (start 212.1128 148.9615) (end 211.8493 149.225) (width 0.254) (layer F.Cu) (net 9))
 (segment (start 215.0347 148.9615) (end 212.1128 148.9615) (width 0.254) (layer F.Cu) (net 9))
 (segment (start 216.764 150.6908) (end 215.0347 148.9615) (width 0.254) (layer F.Cu) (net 9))
 (segment (start 216.764 152.1051) (end 216.764 153.5194) (width 0.254) (layer F.Cu) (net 9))
 (segment (start 217.3763 153.8368) (end 217.7418 153.4713) (width 0.254) (layer B.Cu) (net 9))
 (segment (start 217.3763 156.794) (end 217.3763 153.8368) (width 0.254) (layer B.Cu) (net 9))
 (segment (start 216.764 153.7587) (end 216.751 153.7717) (width 0.254) (layer F.Cu) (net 9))
 (segment (start 216.764 153.5194) (end 216.764 153.7587) (width 0.254) (layer F.Cu) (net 9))
 (segment (start 217.6937 153.5194) (end 216.764 153.5194) (width 0.254) (layer F.Cu) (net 9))
 (segment (start 217.7418 153.4713) (end 217.6937 153.5194) (width 0.254) (layer F.Cu) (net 9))
 (segment (start 215.722 156.794) (end 217.3763 156.794) (width 0.254) (layer B.Cu) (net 9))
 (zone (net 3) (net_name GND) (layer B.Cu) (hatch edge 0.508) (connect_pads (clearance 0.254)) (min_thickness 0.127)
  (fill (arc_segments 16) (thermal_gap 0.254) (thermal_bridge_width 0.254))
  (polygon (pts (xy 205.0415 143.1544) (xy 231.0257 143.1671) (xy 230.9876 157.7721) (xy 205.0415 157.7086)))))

